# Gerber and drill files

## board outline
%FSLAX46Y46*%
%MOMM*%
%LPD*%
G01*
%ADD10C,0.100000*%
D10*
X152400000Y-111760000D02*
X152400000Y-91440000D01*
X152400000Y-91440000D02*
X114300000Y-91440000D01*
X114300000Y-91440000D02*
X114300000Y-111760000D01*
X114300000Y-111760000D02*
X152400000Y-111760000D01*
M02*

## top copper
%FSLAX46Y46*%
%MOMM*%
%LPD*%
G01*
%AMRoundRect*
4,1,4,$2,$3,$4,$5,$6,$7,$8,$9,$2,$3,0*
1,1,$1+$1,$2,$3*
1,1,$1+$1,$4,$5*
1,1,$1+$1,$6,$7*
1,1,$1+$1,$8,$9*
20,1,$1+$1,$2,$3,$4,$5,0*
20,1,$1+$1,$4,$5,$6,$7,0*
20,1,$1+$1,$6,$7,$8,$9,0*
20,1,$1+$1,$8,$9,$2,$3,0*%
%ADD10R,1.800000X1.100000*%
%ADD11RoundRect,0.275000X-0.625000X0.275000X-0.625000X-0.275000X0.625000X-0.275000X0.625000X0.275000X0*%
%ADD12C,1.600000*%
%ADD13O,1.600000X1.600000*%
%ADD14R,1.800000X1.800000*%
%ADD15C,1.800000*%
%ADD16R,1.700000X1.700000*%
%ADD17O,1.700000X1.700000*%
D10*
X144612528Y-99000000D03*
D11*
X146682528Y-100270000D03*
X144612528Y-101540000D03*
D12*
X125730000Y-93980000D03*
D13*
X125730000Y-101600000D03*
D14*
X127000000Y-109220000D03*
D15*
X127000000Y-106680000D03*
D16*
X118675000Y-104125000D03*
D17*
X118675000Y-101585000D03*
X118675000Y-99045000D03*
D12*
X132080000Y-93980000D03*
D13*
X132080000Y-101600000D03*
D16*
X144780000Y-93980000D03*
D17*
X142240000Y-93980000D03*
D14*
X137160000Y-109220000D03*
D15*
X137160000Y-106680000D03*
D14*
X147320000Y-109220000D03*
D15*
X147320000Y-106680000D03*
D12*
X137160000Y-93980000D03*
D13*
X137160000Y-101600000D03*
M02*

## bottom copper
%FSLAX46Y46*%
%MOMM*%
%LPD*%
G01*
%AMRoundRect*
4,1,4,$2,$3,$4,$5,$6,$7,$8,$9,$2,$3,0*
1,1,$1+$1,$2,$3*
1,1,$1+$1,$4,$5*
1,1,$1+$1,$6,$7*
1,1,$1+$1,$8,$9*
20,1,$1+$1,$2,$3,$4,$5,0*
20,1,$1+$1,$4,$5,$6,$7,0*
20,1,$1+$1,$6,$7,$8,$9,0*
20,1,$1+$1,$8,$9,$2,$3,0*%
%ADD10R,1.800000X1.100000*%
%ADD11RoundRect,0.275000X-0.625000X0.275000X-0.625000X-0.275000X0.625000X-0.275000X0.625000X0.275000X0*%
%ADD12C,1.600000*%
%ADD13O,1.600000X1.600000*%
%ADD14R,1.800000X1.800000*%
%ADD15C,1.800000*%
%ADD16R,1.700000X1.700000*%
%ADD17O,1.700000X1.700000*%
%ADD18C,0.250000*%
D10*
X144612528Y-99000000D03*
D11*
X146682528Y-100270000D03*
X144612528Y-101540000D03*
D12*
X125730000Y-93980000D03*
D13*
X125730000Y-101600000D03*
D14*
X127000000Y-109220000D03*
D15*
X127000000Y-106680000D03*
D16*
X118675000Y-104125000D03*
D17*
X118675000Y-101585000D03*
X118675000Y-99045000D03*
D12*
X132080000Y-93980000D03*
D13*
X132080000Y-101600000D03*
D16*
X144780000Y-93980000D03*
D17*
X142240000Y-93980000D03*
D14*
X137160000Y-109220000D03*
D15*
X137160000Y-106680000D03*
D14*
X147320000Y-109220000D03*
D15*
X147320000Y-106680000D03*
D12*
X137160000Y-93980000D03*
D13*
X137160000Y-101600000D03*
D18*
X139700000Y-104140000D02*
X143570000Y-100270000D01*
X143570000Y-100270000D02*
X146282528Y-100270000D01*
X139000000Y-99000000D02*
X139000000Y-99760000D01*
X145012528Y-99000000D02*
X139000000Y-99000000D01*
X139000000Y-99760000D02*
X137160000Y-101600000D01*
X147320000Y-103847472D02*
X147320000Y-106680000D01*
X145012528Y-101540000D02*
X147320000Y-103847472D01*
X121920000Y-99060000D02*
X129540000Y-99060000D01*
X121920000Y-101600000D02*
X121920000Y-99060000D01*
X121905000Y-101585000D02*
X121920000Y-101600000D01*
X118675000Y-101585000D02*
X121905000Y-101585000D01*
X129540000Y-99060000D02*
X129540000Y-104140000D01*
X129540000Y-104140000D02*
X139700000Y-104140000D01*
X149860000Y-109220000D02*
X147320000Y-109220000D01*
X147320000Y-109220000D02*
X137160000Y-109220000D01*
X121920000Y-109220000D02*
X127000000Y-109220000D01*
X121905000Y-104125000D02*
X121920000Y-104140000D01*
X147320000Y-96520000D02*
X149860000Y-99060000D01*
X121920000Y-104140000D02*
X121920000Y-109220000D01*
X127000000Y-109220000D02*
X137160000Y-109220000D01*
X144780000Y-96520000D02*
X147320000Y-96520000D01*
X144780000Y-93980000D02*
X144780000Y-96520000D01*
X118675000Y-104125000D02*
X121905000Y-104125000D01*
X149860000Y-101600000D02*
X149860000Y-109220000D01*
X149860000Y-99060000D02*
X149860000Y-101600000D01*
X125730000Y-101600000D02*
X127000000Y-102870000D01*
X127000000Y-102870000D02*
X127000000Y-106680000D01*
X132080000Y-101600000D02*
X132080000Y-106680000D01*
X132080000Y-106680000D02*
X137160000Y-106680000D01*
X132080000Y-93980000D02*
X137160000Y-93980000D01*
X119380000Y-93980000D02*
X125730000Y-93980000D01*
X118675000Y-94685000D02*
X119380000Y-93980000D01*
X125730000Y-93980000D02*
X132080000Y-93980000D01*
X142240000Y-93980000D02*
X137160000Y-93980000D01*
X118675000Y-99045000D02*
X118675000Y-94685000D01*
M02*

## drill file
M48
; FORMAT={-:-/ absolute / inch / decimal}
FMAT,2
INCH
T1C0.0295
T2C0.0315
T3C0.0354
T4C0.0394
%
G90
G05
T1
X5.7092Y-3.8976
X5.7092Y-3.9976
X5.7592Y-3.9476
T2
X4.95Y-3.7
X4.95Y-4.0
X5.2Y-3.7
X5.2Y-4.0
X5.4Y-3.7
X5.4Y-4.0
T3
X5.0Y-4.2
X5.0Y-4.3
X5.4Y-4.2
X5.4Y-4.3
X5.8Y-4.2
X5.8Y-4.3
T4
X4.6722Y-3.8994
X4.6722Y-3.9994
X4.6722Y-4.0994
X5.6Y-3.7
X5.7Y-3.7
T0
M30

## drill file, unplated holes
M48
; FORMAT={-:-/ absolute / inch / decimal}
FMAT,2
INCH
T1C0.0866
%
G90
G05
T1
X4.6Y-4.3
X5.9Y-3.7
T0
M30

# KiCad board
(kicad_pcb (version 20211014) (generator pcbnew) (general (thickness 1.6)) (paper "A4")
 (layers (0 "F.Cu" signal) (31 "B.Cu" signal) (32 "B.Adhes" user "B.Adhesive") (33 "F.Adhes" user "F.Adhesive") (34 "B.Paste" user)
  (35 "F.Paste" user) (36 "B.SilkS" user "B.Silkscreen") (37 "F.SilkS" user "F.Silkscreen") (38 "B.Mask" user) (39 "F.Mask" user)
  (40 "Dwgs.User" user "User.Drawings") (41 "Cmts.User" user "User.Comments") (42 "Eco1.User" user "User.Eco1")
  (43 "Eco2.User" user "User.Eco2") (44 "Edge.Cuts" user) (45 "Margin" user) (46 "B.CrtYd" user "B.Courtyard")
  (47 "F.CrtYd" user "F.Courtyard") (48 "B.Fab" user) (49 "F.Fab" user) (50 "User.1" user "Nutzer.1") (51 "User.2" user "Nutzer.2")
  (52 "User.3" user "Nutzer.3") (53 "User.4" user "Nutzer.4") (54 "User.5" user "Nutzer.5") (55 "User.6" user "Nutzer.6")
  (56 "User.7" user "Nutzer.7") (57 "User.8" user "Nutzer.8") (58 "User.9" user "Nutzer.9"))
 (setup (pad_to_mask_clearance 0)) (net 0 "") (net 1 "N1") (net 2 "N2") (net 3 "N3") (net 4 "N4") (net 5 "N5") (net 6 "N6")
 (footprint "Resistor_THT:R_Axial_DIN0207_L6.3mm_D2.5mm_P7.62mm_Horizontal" (layer "F.Cu") (at 125.73 93.98 -90)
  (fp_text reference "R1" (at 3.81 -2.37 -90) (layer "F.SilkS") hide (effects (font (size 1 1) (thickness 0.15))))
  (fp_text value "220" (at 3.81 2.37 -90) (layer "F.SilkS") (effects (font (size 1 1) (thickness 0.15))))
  (pad "1" thru_hole circle (at 0 0 270) (size 1.6 1.6) (drill 0.8) (layers *.Cu *.Mask) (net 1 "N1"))
  (pad "2" thru_hole oval (at 7.62 0 270) (size 1.6 1.6) (drill 0.8) (layers *.Cu *.Mask) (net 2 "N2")))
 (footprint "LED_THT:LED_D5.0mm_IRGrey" (layer "F.Cu") (at 127 109.22 90)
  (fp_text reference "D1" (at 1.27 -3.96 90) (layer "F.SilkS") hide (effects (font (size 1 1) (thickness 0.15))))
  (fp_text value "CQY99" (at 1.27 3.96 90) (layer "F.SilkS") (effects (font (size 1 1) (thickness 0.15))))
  (pad "1" thru_hole rect (at 0 0 90) (size 1.8 1.8) (drill 0.9) (layers *.Cu *.Mask) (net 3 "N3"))
  (pad "2" thru_hole circle (at 2.54 0 90) (size 1.8 1.8) (drill 0.9) (layers *.Cu *.Mask) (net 2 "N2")))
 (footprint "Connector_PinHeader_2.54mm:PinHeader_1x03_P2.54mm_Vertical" (layer "F.Cu") (at 118.675 104.125 180)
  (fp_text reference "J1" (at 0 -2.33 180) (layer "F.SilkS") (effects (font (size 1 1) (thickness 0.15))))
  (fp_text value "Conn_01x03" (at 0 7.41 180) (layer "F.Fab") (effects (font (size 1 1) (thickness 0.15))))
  (pad "1" thru_hole rect (at 0 0 180) (size 1.7 1.7) (drill 1) (layers *.Cu *.Mask) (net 3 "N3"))
  (pad "2" thru_hole oval (at 0 2.54 180) (size 1.7 1.7) (drill 1) (layers *.Cu *.Mask) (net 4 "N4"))
  (pad "3" thru_hole oval (at 0 5.08 180) (size 1.7 1.7) (drill 1) (layers *.Cu *.Mask) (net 1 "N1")))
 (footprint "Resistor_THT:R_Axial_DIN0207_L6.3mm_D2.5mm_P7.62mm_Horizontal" (layer "F.Cu") (at 132.08 93.98 -90)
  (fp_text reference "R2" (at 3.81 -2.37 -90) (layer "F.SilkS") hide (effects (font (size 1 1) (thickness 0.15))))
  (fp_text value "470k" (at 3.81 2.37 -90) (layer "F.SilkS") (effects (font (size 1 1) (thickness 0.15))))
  (pad "1" thru_hole circle (at 0 0 270) (size 1.6 1.6) (drill 0.8) (layers *.Cu *.Mask) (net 1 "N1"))
  (pad "2" thru_hole oval (at 7.62 0 270) (size 1.6 1.6) (drill 0.8) (layers *.Cu *.Mask) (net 4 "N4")))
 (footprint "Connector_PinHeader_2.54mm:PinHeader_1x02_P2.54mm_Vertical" (layer "F.Cu") (at 144.78 93.98 -90)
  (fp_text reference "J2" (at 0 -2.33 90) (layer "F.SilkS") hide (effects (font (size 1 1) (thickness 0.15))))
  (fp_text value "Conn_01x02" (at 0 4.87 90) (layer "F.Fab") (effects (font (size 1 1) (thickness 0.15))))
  (pad "1" thru_hole rect (at 0 0 270) (size 1.7 1.7) (drill 1) (layers *.Cu *.Mask) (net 3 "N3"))
  (pad "2" thru_hole oval (at 0 2.54 270) (size 1.7 1.7) (drill 1) (layers *.Cu *.Mask) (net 1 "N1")))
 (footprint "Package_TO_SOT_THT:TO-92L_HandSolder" (layer "F.Cu") (at 145.012528 99 -90)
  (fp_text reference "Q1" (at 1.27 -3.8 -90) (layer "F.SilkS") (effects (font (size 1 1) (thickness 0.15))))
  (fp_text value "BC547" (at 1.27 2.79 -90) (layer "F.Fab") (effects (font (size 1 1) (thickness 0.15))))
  (pad "1" thru_hole rect (at 0 0 270) (size 1.1 1.8) (drill 0.75 (offset 0 0.4)) (layers *.Cu *.Mask) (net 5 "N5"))
  (pad "2" thru_hole roundrect (at 1.27 -1.27 270) (size 1.1 1.8) (drill 0.75 (offset 0 -0.4)) (layers *.Cu *.Mask) (roundrect_rratio 0.25)
   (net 4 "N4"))
  (pad "3" thru_hole roundrect (at 2.54 0 270) (size 1.1 1.8) (drill 0.75 (offset 0 0.4)) (layers *.Cu *.Mask) (roundrect_rratio 0.25)
   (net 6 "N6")))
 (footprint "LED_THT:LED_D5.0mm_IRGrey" (layer "F.Cu") (at 137.16 109.22 90)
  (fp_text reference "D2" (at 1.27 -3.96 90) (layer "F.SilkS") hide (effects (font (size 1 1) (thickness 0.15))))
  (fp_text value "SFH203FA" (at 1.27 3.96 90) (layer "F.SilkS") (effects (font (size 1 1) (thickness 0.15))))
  (pad "1" thru_hole rect (at 0 0 90) (size 1.8 1.8) (drill 0.9) (layers *.Cu *.Mask) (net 3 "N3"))
  (pad "2" thru_hole circle (at 2.54 0 90) (size 1.8 1.8) (drill 0.9) (layers *.Cu *.Mask) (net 4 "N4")))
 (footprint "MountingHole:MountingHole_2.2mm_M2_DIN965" (layer "F.Cu") (at 149.86 93.98 180)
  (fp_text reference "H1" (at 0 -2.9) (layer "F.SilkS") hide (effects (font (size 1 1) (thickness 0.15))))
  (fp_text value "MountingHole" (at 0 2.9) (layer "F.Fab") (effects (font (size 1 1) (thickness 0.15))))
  (pad "" np_thru_hole circle (at 0 0 180) (size 2.2 2.2) (drill 2.2) (layers *.Cu *.Mask)))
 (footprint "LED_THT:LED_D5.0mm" (layer "F.Cu") (at 147.32 109.22 90)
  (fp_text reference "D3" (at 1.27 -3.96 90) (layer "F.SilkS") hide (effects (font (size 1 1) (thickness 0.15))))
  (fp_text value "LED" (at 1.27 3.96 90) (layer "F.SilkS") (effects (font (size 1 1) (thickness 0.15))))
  (pad "1" thru_hole rect (at 0 0 90) (size 1.8 1.8) (drill 0.9) (layers *.Cu *.Mask) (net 3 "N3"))
  (pad "2" thru_hole circle (at 2.54 0 90) (size 1.8 1.8) (drill 0.9) (layers *.Cu *.Mask) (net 6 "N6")))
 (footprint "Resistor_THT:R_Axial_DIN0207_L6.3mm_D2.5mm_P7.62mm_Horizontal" (layer "F.Cu") (at 137.16 93.98 -90)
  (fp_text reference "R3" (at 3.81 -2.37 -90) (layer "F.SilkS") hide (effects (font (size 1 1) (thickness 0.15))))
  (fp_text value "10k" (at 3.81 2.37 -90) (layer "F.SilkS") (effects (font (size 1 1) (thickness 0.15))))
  (pad "1" thru_hole circle (at 0 0 270) (size 1.6 1.6) (drill 0.8) (layers *.Cu *.Mask) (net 1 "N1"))
  (pad "2" thru_hole oval (at 7.62 0 270) (size 1.6 1.6) (drill 0.8) (layers *.Cu *.Mask) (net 5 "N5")))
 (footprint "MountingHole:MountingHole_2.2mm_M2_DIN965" (layer "F.Cu") (at 116.84 109.22)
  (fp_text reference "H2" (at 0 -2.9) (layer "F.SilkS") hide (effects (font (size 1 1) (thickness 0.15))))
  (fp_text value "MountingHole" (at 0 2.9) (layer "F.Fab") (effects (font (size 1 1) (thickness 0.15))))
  (pad "" np_thru_hole circle (at 0 0) (size 2.2 2.2) (drill 2.2) (layers *.Cu *.Mask)))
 (gr_line (start 152.4 111.76) (end 152.4 91.44) (layer "Edge.Cuts") (width 0.1))
 (gr_line (start 152.4 91.44) (end 114.3 91.44) (layer "Edge.Cuts") (width 0.1))
 (gr_line (start 114.3 91.44) (end 114.3 111.76) (layer "Edge.Cuts") (width 0.1))
 (gr_line (start 114.3 111.76) (end 152.4 111.76) (layer "Edge.Cuts") (width 0.1))
 (segment (start 149.86 109.22) (end 147.32 109.22) (width 0.25) (layer "B.Cu") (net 3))
 (segment (start 147.32 109.22) (end 137.16 109.22) (width 0.25) (layer "B.Cu") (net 3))
 (segment (start 121.92 109.22) (end 127 109.22) (width 0.25) (layer "B.Cu") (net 3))
 (segment (start 121.905 104.125) (end 121.92 104.14) (width 0.25) (layer "B.Cu") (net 3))
 (segment (start 147.32 96.52) (end 149.86 99.06) (width 0.25) (layer "B.Cu") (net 3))
 (segment (start 121.92 104.14) (end 121.92 109.22) (width 0.25) (layer "B.Cu") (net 3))
 (segment (start 127 109.22) (end 137.16 109.22) (width 0.25) (layer "B.Cu") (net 3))
 (segment (start 144.78 96.52) (end 147.32 96.52) (width 0.25) (layer "B.Cu") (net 3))
 (segment (start 144.78 93.98) (end 144.78 96.52) (width 0.25) (layer "B.Cu") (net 3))
 (segment (start 118.675 104.125) (end 121.905 104.125) (width 0.25) (layer "B.Cu") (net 3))
 (segment (start 149.86 101.6) (end 149.86 109.22) (width 0.25) (layer "B.Cu") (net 3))
 (segment (start 149.86 99.06) (end 149.86 101.6) (width 0.25) (layer "B.Cu") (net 3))
 (segment (start 125.73 101.6) (end 127 102.87) (width 0.25) (layer "B.Cu") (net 2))
 (segment (start 127 102.87) (end 127 106.68) (width 0.25) (layer "B.Cu") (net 2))
 (segment (start 143.57 100.27) (end 146.282528 100.27) (width 0.25) (layer "B.Cu") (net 4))
 (segment (start 121.92 99.06) (end 129.54 99.06) (width 0.25) (layer "B.Cu") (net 4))
 (segment (start 129.54 99.06) (end 129.54 104.14) (width 0.25) (layer "B.Cu") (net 4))
 (segment (start 121.92 101.6) (end 121.92 99.06) (width 0.25) (layer "B.Cu") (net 4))
 (segment (start 132.08 101.6) (end 132.08 106.68) (width 0.25) (layer "B.Cu") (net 4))
 (segment (start 118.675 101.585) (end 121.905 101.585) (width 0.25) (layer "B.Cu") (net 4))
 (segment (start 121.905 101.585) (end 121.92 101.6) (width 0.25) (layer "B.Cu") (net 4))
 (segment (start 139.7 104.14) (end 143.57 100.27) (width 0.25) (layer "B.Cu") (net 4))
 (segment (start 129.54 104.14) (end 139.7 104.14) (width 0.25) (layer "B.Cu") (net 4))
 (segment (start 132.08 106.68) (end 137.16 106.68) (width 0.25) (layer "B.Cu") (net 4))
 (segment (start 132.08 93.98) (end 137.16 93.98) (width 0.25) (layer "B.Cu") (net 1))
 (segment (start 119.38 93.98) (end 125.73 93.98) (width 0.25) (layer "B.Cu") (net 1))
 (segment (start 118.675 94.685) (end 119.38 93.98) (width 0.25) (layer "B.Cu") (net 1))
 (segment (start 125.73 93.98) (end 132.08 93.98) (width 0.25) (layer "B.Cu") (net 1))
 (segment (start 142.24 93.98) (end 137.16 93.98) (width 0.25) (layer "B.Cu") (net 1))
 (segment (start 118.675 99.045) (end 118.675 94.685) (width 0.25) (layer "B.Cu") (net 1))
 (segment (start 139 99) (end 139 99.76) (width 0.25) (layer "B.Cu") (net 5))
 (segment (start 145.012528 99) (end 139 99) (width 0.25) (layer "B.Cu") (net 5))
 (segment (start 139 99.76) (end 137.16 101.6) (width 0.25) (layer "B.Cu") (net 5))
 (segment (start 145.012528 101.54) (end 147.32 103.847472) (width 0.25) (layer "B.Cu") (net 6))
 (segment (start 147.32 103.847472) (end 147.32 106.68) (width 0.25) (layer "B.Cu") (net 6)))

